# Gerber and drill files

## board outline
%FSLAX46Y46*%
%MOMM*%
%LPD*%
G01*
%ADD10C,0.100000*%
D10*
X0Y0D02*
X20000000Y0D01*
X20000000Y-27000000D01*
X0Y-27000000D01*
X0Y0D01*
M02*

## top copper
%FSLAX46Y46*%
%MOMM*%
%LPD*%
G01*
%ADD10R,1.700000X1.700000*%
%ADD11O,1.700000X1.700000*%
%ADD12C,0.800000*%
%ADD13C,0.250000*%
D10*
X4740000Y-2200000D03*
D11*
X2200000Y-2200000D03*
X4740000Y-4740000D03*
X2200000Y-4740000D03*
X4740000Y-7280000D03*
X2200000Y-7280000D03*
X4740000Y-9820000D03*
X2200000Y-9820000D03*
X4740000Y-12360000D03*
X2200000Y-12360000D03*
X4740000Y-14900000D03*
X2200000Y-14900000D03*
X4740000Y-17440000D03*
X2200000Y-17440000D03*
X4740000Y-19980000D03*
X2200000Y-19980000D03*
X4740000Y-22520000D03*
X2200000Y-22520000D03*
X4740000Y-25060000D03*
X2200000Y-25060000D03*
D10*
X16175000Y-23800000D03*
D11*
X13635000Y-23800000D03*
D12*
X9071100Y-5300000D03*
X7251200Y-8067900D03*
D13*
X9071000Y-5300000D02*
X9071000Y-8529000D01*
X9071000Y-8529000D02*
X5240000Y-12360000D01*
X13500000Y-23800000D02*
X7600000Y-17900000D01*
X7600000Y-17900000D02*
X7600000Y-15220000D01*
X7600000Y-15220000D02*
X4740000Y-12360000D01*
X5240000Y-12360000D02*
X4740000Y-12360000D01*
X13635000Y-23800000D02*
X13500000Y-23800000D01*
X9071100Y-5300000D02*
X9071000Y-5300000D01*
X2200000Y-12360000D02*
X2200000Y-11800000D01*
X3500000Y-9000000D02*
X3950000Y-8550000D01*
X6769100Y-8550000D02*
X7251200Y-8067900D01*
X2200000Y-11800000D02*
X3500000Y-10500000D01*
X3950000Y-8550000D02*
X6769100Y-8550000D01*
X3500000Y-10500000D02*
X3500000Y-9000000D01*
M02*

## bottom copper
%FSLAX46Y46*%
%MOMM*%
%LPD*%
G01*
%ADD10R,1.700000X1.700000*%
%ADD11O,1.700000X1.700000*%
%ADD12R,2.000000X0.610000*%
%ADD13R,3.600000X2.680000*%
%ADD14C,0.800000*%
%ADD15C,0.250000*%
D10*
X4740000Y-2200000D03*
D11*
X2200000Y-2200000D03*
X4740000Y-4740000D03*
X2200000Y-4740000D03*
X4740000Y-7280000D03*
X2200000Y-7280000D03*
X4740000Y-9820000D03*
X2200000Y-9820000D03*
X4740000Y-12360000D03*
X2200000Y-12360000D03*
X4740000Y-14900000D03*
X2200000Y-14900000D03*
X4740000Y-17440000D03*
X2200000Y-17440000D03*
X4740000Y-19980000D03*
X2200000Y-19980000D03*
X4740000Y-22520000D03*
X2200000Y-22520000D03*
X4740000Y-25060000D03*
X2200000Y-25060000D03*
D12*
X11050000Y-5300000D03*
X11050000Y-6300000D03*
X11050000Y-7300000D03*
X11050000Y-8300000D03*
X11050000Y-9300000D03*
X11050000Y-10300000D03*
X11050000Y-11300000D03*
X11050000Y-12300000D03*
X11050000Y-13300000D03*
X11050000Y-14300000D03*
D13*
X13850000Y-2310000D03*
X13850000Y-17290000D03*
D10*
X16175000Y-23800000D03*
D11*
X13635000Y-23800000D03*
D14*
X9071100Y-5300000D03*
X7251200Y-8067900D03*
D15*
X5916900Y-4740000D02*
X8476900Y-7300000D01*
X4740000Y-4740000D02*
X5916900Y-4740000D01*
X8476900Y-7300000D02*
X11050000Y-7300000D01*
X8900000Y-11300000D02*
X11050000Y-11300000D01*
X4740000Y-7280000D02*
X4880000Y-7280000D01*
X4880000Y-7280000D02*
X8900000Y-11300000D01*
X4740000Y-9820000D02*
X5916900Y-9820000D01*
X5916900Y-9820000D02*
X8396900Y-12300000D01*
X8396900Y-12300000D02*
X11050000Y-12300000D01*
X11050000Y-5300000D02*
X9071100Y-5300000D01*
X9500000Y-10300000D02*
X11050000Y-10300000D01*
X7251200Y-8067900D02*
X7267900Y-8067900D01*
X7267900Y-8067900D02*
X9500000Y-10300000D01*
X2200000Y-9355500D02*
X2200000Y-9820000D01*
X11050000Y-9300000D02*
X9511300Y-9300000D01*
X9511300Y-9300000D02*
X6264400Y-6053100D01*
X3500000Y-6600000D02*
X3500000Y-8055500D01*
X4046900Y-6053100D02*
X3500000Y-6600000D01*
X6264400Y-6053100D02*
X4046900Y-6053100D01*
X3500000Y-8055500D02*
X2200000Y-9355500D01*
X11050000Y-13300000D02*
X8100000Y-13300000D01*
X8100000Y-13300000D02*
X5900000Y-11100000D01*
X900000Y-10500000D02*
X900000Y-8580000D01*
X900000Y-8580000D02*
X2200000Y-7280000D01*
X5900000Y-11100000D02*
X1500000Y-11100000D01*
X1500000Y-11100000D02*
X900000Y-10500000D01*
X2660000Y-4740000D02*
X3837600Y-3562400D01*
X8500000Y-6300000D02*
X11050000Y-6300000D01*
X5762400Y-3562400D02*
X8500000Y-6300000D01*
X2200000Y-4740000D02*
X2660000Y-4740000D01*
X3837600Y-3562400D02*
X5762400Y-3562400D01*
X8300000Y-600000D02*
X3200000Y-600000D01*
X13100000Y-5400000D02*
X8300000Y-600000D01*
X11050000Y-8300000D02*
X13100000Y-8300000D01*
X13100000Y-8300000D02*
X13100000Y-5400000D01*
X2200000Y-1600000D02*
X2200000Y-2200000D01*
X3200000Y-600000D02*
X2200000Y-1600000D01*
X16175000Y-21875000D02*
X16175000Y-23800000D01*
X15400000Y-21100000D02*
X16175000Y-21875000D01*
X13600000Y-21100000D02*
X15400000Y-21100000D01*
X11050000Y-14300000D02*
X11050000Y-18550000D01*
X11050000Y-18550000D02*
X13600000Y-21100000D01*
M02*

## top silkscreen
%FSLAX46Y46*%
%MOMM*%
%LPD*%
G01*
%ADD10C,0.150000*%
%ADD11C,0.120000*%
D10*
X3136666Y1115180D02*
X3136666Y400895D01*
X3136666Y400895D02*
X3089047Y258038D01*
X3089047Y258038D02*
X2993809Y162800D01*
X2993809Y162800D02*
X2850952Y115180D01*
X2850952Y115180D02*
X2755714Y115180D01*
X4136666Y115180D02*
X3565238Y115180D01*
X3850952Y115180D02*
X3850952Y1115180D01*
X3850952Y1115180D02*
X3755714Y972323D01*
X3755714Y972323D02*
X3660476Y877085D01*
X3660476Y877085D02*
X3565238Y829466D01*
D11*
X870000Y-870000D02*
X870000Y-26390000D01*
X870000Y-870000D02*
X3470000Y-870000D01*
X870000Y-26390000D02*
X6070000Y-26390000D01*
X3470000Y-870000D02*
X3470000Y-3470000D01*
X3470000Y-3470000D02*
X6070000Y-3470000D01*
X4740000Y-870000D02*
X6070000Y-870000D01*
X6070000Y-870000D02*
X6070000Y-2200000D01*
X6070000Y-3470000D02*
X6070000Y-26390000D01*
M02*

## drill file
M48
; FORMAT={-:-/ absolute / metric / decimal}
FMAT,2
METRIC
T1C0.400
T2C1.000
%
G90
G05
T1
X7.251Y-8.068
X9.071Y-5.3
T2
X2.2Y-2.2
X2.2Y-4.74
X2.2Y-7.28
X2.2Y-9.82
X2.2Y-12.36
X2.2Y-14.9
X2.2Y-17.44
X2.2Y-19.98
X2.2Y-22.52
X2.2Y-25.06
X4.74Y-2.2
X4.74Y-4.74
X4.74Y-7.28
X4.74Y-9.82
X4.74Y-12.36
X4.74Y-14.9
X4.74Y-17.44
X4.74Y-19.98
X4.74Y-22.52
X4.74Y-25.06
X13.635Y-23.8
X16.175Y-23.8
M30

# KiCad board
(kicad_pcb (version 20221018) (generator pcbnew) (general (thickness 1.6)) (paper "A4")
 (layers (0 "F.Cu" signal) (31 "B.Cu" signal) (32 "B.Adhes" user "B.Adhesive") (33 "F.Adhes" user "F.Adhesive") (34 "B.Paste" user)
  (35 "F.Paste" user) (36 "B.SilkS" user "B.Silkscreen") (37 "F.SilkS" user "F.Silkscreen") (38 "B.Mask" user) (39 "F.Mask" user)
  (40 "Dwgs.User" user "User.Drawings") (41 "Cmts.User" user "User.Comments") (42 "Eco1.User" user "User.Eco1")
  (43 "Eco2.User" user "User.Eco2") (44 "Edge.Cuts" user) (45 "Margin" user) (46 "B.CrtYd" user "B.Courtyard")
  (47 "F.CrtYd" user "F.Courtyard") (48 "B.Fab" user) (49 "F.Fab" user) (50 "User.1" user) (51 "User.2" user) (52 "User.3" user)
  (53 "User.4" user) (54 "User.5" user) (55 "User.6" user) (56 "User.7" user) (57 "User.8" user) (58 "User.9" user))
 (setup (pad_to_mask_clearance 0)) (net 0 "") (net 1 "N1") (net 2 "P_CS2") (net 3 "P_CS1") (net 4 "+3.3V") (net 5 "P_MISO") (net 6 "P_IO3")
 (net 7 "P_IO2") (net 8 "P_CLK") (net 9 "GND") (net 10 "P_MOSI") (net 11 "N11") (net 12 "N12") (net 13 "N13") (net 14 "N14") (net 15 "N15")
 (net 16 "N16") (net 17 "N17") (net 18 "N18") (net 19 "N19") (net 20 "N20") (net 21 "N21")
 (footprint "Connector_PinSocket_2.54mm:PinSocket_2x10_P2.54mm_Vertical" (layer "F.Cu") (at 4.74 2.2)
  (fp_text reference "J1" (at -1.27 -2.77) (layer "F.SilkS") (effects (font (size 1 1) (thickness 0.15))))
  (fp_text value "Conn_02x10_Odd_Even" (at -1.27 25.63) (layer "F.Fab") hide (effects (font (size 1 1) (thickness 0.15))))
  (fp_line (start -3.87 -1.33) (end -3.87 24.19) (stroke (width 0.12) (type solid)) (layer "F.SilkS"))
  (fp_line (start -3.87 -1.33) (end -1.27 -1.33) (stroke (width 0.12) (type solid)) (layer "F.SilkS"))
  (fp_line (start -3.87 24.19) (end 1.33 24.19) (stroke (width 0.12) (type solid)) (layer "F.SilkS"))
  (fp_line (start -1.27 -1.33) (end -1.27 1.27) (stroke (width 0.12) (type solid)) (layer "F.SilkS"))
  (fp_line (start -1.27 1.27) (end 1.33 1.27) (stroke (width 0.12) (type solid)) (layer "F.SilkS"))
  (fp_line (start 0 -1.33) (end 1.33 -1.33) (stroke (width 0.12) (type solid)) (layer "F.SilkS"))
  (fp_line (start 1.33 -1.33) (end 1.33 0) (stroke (width 0.12) (type solid)) (layer "F.SilkS"))
  (fp_line (start 1.33 1.27) (end 1.33 24.19) (stroke (width 0.12) (type solid)) (layer "F.SilkS"))
  (pad "1" thru_hole rect (at 0 0) (size 1.7 1.7) (drill 1) (layers "*.Cu" "*.Mask") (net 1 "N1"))
  (pad "2" thru_hole oval (at -2.54 0) (size 1.7 1.7) (drill 1) (layers "*.Cu" "*.Mask") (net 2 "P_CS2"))
  (pad "3" thru_hole oval (at 0 2.54) (size 1.7 1.7) (drill 1) (layers "*.Cu" "*.Mask") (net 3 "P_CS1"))
  (pad "4" thru_hole oval (at -2.54 2.54) (size 1.7 1.7) (drill 1) (layers "*.Cu" "*.Mask") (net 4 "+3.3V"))
  (pad "5" thru_hole oval (at 0 5.08) (size 1.7 1.7) (drill 1) (layers "*.Cu" "*.Mask") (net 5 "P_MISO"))
  (pad "6" thru_hole oval (at -2.54 5.08) (size 1.7 1.7) (drill 1) (layers "*.Cu" "*.Mask") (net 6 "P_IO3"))
  (pad "7" thru_hole oval (at 0 7.62) (size 1.7 1.7) (drill 1) (layers "*.Cu" "*.Mask") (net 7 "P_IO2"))
  (pad "8" thru_hole oval (at -2.54 7.62) (size 1.7 1.7) (drill 1) (layers "*.Cu" "*.Mask") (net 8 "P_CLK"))
  (pad "9" thru_hole oval (at 0 10.16) (size 1.7 1.7) (drill 1) (layers "*.Cu" "*.Mask") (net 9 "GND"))
  (pad "10" thru_hole oval (at -2.54 10.16) (size 1.7 1.7) (drill 1) (layers "*.Cu" "*.Mask") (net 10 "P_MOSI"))
  (pad "11" thru_hole oval (at 0 12.7) (size 1.7 1.7) (drill 1) (layers "*.Cu" "*.Mask") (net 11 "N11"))
  (pad "12" thru_hole oval (at -2.54 12.7) (size 1.7 1.7) (drill 1) (layers "*.Cu" "*.Mask") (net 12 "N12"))
  (pad "13" thru_hole oval (at 0 15.24) (size 1.7 1.7) (drill 1) (layers "*.Cu" "*.Mask") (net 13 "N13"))
  (pad "14" thru_hole oval (at -2.54 15.24) (size 1.7 1.7) (drill 1) (layers "*.Cu" "*.Mask") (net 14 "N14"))
  (pad "15" thru_hole oval (at 0 17.78) (size 1.7 1.7) (drill 1) (layers "*.Cu" "*.Mask") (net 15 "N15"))
  (pad "16" thru_hole oval (at -2.54 17.78) (size 1.7 1.7) (drill 1) (layers "*.Cu" "*.Mask") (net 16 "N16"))
  (pad "17" thru_hole oval (at 0 20.32) (size 1.7 1.7) (drill 1) (layers "*.Cu" "*.Mask") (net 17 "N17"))
  (pad "18" thru_hole oval (at -2.54 20.32) (size 1.7 1.7) (drill 1) (layers "*.Cu" "*.Mask") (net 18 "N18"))
  (pad "19" thru_hole oval (at 0 22.86) (size 1.7 1.7) (drill 1) (layers "*.Cu" "*.Mask") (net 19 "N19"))
  (pad "20" thru_hole oval (at -2.54 22.86) (size 1.7 1.7) (drill 1) (layers "*.Cu" "*.Mask") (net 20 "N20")))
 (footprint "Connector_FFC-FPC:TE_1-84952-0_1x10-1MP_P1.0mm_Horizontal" (layer "B.Cu") (at 12.85 9.8 -90)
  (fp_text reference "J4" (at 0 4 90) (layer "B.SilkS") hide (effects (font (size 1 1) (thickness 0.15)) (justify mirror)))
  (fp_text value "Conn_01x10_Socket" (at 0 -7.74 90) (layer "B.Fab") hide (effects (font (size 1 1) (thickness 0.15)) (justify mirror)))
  (pad "1" smd rect (at -4.5 1.8 270) (size 0.61 2) (layers "B.Cu" "B.Paste" "B.Mask") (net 9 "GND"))
  (pad "2" smd rect (at -3.5 1.8 270) (size 0.61 2) (layers "B.Cu" "B.Paste" "B.Mask") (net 4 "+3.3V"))
  (pad "3" smd rect (at -2.5 1.8 270) (size 0.61 2) (layers "B.Cu" "B.Paste" "B.Mask") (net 3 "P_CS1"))
  (pad "4" smd rect (at -1.5 1.8 270) (size 0.61 2) (layers "B.Cu" "B.Paste" "B.Mask") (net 2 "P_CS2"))
  (pad "5" smd rect (at -0.5 1.8 270) (size 0.61 2) (layers "B.Cu" "B.Paste" "B.Mask") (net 8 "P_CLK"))
  (pad "6" smd rect (at 0.5 1.8 270) (size 0.61 2) (layers "B.Cu" "B.Paste" "B.Mask") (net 10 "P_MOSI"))
  (pad "7" smd rect (at 1.5 1.8 270) (size 0.61 2) (layers "B.Cu" "B.Paste" "B.Mask") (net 5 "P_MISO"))
  (pad "8" smd rect (at 2.5 1.8 270) (size 0.61 2) (layers "B.Cu" "B.Paste" "B.Mask") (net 7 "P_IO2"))
  (pad "9" smd rect (at 3.5 1.8 270) (size 0.61 2) (layers "B.Cu" "B.Paste" "B.Mask") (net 6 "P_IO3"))
  (pad "10" smd rect (at 4.5 1.8 270) (size 0.61 2) (layers "B.Cu" "B.Paste" "B.Mask") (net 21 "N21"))
  (pad "MP" smd rect (at -7.49 -1 270) (size 2.68 3.6) (layers "B.Cu" "B.Paste" "B.Mask"))
  (pad "MP" smd rect (at 7.49 -1 270) (size 2.68 3.6) (layers "B.Cu" "B.Paste" "B.Mask")))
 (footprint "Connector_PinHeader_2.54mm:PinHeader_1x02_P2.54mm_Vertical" (layer "B.Cu") (at 16.175 23.8 90)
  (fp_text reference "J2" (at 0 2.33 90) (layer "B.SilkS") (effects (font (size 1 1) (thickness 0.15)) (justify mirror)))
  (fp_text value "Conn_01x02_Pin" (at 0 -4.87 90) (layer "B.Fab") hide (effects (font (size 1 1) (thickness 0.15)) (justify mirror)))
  (pad "1" thru_hole rect (at 0 0 90) (size 1.7 1.7) (drill 1) (layers "*.Cu" "*.Mask") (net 21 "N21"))
  (pad "2" thru_hole oval (at 0 -2.54 90) (size 1.7 1.7) (drill 1) (layers "*.Cu" "*.Mask") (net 9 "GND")))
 (gr_rect (start 0 0) (end 20 27) (stroke (width 0.1) (type default)) (fill none) (layer "Edge.Cuts"))
 (segment (start 5.9169 4.74) (end 8.4769 7.3) (width 0.25) (layer "B.Cu") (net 3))
 (segment (start 4.74 4.74) (end 5.9169 4.74) (width 0.25) (layer "B.Cu") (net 3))
 (segment (start 8.4769 7.3) (end 11.05 7.3) (width 0.25) (layer "B.Cu") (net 3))
 (segment (start 8.9 11.3) (end 11.05 11.3) (width 0.25) (layer "B.Cu") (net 5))
 (segment (start 4.74 7.28) (end 4.88 7.28) (width 0.25) (layer "B.Cu") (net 5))
 (segment (start 4.88 7.28) (end 8.9 11.3) (width 0.25) (layer "B.Cu") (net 5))
 (segment (start 4.74 9.82) (end 5.9169 9.82) (width 0.25) (layer "B.Cu") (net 7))
 (segment (start 5.9169 9.82) (end 8.3969 12.3) (width 0.25) (layer "B.Cu") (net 7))
 (segment (start 8.3969 12.3) (end 11.05 12.3) (width 0.25) (layer "B.Cu") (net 7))
 (segment (start 9.071 5.3) (end 9.071 8.529) (width 0.25) (layer "F.Cu") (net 9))
 (segment (start 9.071 8.529) (end 5.24 12.36) (width 0.25) (layer "F.Cu") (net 9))
 (segment (start 13.5 23.8) (end 7.6 17.9) (width 0.25) (layer "F.Cu") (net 9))
 (segment (start 7.6 17.9) (end 7.6 15.22) (width 0.25) (layer "F.Cu") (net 9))
 (segment (start 7.6 15.22) (end 4.74 12.36) (width 0.25) (layer "F.Cu") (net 9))
 (segment (start 5.24 12.36) (end 4.74 12.36) (width 0.25) (layer "F.Cu") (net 9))
 (segment (start 13.635 23.8) (end 13.5 23.8) (width 0.25) (layer "F.Cu") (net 9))
 (segment (start 9.0711 5.3) (end 9.071 5.3) (width 0.25) (layer "F.Cu") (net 9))
 (via (at 9.0711 5.3) (size 0.8) (drill 0.4) (layers "F.Cu" "B.Cu") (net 9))
 (segment (start 11.05 5.3) (end 9.0711 5.3) (width 0.25) (layer "B.Cu") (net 9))
 (segment (start 2.2 12.36) (end 2.2 11.8) (width 0.25) (layer "F.Cu") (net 10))
 (segment (start 3.5 9) (end 3.95 8.55) (width 0.25) (layer "F.Cu") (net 10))
 (segment (start 6.7691 8.55) (end 7.2512 8.0679) (width 0.25) (layer "F.Cu") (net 10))
 (segment (start 2.2 11.8) (end 3.5 10.5) (width 0.25) (layer "F.Cu") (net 10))
 (segment (start 3.95 8.55) (end 6.7691 8.55) (width 0.25) (layer "F.Cu") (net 10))
 (segment (start 3.5 10.5) (end 3.5 9) (width 0.25) (layer "F.Cu") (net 10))
 (via (at 7.2512 8.0679) (size 0.8) (drill 0.4) (layers "F.Cu" "B.Cu") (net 10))
 (segment (start 9.5 10.3) (end 11.05 10.3) (width 0.25) (layer "B.Cu") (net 10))
 (segment (start 7.2512 8.0679) (end 7.2679 8.0679) (width 0.25) (layer "B.Cu") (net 10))
 (segment (start 7.2679 8.0679) (end 9.5 10.3) (width 0.25) (layer "B.Cu") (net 10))
 (segment (start 2.2 9.3555) (end 2.2 9.82) (width 0.25) (layer "B.Cu") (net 8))
 (segment (start 11.05 9.3) (end 9.5113 9.3) (width 0.25) (layer "B.Cu") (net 8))
 (segment (start 9.5113 9.3) (end 6.2644 6.0531) (width 0.25) (layer "B.Cu") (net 8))
 (segment (start 3.5 6.6) (end 3.5 8.0555) (width 0.25) (layer "B.Cu") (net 8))
 (segment (start 4.0469 6.0531) (end 3.5 6.6) (width 0.25) (layer "B.Cu") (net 8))
 (segment (start 6.2644 6.0531) (end 4.0469 6.0531) (width 0.25) (layer "B.Cu") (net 8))
 (segment (start 3.5 8.0555) (end 2.2 9.3555) (width 0.25) (layer "B.Cu") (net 8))
 (segment (start 11.05 13.3) (end 8.1 13.3) (width 0.25) (layer "B.Cu") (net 6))
 (segment (start 8.1 13.3) (end 5.9 11.1) (width 0.25) (layer "B.Cu") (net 6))
 (segment (start 0.9 10.5) (end 0.9 8.58) (width 0.25) (layer "B.Cu") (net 6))
 (segment (start 0.9 8.58) (end 2.2 7.28) (width 0.25) (layer "B.Cu") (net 6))
 (segment (start 5.9 11.1) (end 1.5 11.1) (width 0.25) (layer "B.Cu") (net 6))
 (segment (start 1.5 11.1) (end 0.9 10.5) (width 0.25) (layer "B.Cu") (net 6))
 (segment (start 2.66 4.74) (end 3.8376 3.5624) (width 0.25) (layer "B.Cu") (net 4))
 (segment (start 8.5 6.3) (end 11.05 6.3) (width 0.25) (layer "B.Cu") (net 4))
 (segment (start 5.7624 3.5624) (end 8.5 6.3) (width 0.25) (layer "B.Cu") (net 4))
 (segment (start 2.2 4.74) (end 2.66 4.74) (width 0.25) (layer "B.Cu") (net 4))
 (segment (start 3.8376 3.5624) (end 5.7624 3.5624) (width 0.25) (layer "B.Cu") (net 4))
 (segment (start 8.3 0.6) (end 3.2 0.6) (width 0.25) (layer "B.Cu") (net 2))
 (segment (start 13.1 5.4) (end 8.3 0.6) (width 0.25) (layer "B.Cu") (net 2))
 (segment (start 11.05 8.3) (end 13.1 8.3) (width 0.25) (layer "B.Cu") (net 2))
 (segment (start 13.1 8.3) (end 13.1 5.4) (width 0.25) (layer "B.Cu") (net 2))
 (segment (start 2.2 1.6) (end 2.2 2.2) (width 0.25) (layer "B.Cu") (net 2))
 (segment (start 3.2 0.6) (end 2.2 1.6) (width 0.25) (layer "B.Cu") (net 2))
 (segment (start 16.175 21.875) (end 16.175 23.8) (width 0.25) (layer "B.Cu") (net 21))
 (segment (start 15.4 21.1) (end 16.175 21.875) (width 0.25) (layer "B.Cu") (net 21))
 (segment (start 13.6 21.1) (end 15.4 21.1) (width 0.25) (layer "B.Cu") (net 21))
 (segment (start 11.05 14.3) (end 11.05 18.55) (width 0.25) (layer "B.Cu") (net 21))
 (segment (start 11.05 18.55) (end 13.6 21.1) (width 0.25) (layer "B.Cu") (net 21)))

